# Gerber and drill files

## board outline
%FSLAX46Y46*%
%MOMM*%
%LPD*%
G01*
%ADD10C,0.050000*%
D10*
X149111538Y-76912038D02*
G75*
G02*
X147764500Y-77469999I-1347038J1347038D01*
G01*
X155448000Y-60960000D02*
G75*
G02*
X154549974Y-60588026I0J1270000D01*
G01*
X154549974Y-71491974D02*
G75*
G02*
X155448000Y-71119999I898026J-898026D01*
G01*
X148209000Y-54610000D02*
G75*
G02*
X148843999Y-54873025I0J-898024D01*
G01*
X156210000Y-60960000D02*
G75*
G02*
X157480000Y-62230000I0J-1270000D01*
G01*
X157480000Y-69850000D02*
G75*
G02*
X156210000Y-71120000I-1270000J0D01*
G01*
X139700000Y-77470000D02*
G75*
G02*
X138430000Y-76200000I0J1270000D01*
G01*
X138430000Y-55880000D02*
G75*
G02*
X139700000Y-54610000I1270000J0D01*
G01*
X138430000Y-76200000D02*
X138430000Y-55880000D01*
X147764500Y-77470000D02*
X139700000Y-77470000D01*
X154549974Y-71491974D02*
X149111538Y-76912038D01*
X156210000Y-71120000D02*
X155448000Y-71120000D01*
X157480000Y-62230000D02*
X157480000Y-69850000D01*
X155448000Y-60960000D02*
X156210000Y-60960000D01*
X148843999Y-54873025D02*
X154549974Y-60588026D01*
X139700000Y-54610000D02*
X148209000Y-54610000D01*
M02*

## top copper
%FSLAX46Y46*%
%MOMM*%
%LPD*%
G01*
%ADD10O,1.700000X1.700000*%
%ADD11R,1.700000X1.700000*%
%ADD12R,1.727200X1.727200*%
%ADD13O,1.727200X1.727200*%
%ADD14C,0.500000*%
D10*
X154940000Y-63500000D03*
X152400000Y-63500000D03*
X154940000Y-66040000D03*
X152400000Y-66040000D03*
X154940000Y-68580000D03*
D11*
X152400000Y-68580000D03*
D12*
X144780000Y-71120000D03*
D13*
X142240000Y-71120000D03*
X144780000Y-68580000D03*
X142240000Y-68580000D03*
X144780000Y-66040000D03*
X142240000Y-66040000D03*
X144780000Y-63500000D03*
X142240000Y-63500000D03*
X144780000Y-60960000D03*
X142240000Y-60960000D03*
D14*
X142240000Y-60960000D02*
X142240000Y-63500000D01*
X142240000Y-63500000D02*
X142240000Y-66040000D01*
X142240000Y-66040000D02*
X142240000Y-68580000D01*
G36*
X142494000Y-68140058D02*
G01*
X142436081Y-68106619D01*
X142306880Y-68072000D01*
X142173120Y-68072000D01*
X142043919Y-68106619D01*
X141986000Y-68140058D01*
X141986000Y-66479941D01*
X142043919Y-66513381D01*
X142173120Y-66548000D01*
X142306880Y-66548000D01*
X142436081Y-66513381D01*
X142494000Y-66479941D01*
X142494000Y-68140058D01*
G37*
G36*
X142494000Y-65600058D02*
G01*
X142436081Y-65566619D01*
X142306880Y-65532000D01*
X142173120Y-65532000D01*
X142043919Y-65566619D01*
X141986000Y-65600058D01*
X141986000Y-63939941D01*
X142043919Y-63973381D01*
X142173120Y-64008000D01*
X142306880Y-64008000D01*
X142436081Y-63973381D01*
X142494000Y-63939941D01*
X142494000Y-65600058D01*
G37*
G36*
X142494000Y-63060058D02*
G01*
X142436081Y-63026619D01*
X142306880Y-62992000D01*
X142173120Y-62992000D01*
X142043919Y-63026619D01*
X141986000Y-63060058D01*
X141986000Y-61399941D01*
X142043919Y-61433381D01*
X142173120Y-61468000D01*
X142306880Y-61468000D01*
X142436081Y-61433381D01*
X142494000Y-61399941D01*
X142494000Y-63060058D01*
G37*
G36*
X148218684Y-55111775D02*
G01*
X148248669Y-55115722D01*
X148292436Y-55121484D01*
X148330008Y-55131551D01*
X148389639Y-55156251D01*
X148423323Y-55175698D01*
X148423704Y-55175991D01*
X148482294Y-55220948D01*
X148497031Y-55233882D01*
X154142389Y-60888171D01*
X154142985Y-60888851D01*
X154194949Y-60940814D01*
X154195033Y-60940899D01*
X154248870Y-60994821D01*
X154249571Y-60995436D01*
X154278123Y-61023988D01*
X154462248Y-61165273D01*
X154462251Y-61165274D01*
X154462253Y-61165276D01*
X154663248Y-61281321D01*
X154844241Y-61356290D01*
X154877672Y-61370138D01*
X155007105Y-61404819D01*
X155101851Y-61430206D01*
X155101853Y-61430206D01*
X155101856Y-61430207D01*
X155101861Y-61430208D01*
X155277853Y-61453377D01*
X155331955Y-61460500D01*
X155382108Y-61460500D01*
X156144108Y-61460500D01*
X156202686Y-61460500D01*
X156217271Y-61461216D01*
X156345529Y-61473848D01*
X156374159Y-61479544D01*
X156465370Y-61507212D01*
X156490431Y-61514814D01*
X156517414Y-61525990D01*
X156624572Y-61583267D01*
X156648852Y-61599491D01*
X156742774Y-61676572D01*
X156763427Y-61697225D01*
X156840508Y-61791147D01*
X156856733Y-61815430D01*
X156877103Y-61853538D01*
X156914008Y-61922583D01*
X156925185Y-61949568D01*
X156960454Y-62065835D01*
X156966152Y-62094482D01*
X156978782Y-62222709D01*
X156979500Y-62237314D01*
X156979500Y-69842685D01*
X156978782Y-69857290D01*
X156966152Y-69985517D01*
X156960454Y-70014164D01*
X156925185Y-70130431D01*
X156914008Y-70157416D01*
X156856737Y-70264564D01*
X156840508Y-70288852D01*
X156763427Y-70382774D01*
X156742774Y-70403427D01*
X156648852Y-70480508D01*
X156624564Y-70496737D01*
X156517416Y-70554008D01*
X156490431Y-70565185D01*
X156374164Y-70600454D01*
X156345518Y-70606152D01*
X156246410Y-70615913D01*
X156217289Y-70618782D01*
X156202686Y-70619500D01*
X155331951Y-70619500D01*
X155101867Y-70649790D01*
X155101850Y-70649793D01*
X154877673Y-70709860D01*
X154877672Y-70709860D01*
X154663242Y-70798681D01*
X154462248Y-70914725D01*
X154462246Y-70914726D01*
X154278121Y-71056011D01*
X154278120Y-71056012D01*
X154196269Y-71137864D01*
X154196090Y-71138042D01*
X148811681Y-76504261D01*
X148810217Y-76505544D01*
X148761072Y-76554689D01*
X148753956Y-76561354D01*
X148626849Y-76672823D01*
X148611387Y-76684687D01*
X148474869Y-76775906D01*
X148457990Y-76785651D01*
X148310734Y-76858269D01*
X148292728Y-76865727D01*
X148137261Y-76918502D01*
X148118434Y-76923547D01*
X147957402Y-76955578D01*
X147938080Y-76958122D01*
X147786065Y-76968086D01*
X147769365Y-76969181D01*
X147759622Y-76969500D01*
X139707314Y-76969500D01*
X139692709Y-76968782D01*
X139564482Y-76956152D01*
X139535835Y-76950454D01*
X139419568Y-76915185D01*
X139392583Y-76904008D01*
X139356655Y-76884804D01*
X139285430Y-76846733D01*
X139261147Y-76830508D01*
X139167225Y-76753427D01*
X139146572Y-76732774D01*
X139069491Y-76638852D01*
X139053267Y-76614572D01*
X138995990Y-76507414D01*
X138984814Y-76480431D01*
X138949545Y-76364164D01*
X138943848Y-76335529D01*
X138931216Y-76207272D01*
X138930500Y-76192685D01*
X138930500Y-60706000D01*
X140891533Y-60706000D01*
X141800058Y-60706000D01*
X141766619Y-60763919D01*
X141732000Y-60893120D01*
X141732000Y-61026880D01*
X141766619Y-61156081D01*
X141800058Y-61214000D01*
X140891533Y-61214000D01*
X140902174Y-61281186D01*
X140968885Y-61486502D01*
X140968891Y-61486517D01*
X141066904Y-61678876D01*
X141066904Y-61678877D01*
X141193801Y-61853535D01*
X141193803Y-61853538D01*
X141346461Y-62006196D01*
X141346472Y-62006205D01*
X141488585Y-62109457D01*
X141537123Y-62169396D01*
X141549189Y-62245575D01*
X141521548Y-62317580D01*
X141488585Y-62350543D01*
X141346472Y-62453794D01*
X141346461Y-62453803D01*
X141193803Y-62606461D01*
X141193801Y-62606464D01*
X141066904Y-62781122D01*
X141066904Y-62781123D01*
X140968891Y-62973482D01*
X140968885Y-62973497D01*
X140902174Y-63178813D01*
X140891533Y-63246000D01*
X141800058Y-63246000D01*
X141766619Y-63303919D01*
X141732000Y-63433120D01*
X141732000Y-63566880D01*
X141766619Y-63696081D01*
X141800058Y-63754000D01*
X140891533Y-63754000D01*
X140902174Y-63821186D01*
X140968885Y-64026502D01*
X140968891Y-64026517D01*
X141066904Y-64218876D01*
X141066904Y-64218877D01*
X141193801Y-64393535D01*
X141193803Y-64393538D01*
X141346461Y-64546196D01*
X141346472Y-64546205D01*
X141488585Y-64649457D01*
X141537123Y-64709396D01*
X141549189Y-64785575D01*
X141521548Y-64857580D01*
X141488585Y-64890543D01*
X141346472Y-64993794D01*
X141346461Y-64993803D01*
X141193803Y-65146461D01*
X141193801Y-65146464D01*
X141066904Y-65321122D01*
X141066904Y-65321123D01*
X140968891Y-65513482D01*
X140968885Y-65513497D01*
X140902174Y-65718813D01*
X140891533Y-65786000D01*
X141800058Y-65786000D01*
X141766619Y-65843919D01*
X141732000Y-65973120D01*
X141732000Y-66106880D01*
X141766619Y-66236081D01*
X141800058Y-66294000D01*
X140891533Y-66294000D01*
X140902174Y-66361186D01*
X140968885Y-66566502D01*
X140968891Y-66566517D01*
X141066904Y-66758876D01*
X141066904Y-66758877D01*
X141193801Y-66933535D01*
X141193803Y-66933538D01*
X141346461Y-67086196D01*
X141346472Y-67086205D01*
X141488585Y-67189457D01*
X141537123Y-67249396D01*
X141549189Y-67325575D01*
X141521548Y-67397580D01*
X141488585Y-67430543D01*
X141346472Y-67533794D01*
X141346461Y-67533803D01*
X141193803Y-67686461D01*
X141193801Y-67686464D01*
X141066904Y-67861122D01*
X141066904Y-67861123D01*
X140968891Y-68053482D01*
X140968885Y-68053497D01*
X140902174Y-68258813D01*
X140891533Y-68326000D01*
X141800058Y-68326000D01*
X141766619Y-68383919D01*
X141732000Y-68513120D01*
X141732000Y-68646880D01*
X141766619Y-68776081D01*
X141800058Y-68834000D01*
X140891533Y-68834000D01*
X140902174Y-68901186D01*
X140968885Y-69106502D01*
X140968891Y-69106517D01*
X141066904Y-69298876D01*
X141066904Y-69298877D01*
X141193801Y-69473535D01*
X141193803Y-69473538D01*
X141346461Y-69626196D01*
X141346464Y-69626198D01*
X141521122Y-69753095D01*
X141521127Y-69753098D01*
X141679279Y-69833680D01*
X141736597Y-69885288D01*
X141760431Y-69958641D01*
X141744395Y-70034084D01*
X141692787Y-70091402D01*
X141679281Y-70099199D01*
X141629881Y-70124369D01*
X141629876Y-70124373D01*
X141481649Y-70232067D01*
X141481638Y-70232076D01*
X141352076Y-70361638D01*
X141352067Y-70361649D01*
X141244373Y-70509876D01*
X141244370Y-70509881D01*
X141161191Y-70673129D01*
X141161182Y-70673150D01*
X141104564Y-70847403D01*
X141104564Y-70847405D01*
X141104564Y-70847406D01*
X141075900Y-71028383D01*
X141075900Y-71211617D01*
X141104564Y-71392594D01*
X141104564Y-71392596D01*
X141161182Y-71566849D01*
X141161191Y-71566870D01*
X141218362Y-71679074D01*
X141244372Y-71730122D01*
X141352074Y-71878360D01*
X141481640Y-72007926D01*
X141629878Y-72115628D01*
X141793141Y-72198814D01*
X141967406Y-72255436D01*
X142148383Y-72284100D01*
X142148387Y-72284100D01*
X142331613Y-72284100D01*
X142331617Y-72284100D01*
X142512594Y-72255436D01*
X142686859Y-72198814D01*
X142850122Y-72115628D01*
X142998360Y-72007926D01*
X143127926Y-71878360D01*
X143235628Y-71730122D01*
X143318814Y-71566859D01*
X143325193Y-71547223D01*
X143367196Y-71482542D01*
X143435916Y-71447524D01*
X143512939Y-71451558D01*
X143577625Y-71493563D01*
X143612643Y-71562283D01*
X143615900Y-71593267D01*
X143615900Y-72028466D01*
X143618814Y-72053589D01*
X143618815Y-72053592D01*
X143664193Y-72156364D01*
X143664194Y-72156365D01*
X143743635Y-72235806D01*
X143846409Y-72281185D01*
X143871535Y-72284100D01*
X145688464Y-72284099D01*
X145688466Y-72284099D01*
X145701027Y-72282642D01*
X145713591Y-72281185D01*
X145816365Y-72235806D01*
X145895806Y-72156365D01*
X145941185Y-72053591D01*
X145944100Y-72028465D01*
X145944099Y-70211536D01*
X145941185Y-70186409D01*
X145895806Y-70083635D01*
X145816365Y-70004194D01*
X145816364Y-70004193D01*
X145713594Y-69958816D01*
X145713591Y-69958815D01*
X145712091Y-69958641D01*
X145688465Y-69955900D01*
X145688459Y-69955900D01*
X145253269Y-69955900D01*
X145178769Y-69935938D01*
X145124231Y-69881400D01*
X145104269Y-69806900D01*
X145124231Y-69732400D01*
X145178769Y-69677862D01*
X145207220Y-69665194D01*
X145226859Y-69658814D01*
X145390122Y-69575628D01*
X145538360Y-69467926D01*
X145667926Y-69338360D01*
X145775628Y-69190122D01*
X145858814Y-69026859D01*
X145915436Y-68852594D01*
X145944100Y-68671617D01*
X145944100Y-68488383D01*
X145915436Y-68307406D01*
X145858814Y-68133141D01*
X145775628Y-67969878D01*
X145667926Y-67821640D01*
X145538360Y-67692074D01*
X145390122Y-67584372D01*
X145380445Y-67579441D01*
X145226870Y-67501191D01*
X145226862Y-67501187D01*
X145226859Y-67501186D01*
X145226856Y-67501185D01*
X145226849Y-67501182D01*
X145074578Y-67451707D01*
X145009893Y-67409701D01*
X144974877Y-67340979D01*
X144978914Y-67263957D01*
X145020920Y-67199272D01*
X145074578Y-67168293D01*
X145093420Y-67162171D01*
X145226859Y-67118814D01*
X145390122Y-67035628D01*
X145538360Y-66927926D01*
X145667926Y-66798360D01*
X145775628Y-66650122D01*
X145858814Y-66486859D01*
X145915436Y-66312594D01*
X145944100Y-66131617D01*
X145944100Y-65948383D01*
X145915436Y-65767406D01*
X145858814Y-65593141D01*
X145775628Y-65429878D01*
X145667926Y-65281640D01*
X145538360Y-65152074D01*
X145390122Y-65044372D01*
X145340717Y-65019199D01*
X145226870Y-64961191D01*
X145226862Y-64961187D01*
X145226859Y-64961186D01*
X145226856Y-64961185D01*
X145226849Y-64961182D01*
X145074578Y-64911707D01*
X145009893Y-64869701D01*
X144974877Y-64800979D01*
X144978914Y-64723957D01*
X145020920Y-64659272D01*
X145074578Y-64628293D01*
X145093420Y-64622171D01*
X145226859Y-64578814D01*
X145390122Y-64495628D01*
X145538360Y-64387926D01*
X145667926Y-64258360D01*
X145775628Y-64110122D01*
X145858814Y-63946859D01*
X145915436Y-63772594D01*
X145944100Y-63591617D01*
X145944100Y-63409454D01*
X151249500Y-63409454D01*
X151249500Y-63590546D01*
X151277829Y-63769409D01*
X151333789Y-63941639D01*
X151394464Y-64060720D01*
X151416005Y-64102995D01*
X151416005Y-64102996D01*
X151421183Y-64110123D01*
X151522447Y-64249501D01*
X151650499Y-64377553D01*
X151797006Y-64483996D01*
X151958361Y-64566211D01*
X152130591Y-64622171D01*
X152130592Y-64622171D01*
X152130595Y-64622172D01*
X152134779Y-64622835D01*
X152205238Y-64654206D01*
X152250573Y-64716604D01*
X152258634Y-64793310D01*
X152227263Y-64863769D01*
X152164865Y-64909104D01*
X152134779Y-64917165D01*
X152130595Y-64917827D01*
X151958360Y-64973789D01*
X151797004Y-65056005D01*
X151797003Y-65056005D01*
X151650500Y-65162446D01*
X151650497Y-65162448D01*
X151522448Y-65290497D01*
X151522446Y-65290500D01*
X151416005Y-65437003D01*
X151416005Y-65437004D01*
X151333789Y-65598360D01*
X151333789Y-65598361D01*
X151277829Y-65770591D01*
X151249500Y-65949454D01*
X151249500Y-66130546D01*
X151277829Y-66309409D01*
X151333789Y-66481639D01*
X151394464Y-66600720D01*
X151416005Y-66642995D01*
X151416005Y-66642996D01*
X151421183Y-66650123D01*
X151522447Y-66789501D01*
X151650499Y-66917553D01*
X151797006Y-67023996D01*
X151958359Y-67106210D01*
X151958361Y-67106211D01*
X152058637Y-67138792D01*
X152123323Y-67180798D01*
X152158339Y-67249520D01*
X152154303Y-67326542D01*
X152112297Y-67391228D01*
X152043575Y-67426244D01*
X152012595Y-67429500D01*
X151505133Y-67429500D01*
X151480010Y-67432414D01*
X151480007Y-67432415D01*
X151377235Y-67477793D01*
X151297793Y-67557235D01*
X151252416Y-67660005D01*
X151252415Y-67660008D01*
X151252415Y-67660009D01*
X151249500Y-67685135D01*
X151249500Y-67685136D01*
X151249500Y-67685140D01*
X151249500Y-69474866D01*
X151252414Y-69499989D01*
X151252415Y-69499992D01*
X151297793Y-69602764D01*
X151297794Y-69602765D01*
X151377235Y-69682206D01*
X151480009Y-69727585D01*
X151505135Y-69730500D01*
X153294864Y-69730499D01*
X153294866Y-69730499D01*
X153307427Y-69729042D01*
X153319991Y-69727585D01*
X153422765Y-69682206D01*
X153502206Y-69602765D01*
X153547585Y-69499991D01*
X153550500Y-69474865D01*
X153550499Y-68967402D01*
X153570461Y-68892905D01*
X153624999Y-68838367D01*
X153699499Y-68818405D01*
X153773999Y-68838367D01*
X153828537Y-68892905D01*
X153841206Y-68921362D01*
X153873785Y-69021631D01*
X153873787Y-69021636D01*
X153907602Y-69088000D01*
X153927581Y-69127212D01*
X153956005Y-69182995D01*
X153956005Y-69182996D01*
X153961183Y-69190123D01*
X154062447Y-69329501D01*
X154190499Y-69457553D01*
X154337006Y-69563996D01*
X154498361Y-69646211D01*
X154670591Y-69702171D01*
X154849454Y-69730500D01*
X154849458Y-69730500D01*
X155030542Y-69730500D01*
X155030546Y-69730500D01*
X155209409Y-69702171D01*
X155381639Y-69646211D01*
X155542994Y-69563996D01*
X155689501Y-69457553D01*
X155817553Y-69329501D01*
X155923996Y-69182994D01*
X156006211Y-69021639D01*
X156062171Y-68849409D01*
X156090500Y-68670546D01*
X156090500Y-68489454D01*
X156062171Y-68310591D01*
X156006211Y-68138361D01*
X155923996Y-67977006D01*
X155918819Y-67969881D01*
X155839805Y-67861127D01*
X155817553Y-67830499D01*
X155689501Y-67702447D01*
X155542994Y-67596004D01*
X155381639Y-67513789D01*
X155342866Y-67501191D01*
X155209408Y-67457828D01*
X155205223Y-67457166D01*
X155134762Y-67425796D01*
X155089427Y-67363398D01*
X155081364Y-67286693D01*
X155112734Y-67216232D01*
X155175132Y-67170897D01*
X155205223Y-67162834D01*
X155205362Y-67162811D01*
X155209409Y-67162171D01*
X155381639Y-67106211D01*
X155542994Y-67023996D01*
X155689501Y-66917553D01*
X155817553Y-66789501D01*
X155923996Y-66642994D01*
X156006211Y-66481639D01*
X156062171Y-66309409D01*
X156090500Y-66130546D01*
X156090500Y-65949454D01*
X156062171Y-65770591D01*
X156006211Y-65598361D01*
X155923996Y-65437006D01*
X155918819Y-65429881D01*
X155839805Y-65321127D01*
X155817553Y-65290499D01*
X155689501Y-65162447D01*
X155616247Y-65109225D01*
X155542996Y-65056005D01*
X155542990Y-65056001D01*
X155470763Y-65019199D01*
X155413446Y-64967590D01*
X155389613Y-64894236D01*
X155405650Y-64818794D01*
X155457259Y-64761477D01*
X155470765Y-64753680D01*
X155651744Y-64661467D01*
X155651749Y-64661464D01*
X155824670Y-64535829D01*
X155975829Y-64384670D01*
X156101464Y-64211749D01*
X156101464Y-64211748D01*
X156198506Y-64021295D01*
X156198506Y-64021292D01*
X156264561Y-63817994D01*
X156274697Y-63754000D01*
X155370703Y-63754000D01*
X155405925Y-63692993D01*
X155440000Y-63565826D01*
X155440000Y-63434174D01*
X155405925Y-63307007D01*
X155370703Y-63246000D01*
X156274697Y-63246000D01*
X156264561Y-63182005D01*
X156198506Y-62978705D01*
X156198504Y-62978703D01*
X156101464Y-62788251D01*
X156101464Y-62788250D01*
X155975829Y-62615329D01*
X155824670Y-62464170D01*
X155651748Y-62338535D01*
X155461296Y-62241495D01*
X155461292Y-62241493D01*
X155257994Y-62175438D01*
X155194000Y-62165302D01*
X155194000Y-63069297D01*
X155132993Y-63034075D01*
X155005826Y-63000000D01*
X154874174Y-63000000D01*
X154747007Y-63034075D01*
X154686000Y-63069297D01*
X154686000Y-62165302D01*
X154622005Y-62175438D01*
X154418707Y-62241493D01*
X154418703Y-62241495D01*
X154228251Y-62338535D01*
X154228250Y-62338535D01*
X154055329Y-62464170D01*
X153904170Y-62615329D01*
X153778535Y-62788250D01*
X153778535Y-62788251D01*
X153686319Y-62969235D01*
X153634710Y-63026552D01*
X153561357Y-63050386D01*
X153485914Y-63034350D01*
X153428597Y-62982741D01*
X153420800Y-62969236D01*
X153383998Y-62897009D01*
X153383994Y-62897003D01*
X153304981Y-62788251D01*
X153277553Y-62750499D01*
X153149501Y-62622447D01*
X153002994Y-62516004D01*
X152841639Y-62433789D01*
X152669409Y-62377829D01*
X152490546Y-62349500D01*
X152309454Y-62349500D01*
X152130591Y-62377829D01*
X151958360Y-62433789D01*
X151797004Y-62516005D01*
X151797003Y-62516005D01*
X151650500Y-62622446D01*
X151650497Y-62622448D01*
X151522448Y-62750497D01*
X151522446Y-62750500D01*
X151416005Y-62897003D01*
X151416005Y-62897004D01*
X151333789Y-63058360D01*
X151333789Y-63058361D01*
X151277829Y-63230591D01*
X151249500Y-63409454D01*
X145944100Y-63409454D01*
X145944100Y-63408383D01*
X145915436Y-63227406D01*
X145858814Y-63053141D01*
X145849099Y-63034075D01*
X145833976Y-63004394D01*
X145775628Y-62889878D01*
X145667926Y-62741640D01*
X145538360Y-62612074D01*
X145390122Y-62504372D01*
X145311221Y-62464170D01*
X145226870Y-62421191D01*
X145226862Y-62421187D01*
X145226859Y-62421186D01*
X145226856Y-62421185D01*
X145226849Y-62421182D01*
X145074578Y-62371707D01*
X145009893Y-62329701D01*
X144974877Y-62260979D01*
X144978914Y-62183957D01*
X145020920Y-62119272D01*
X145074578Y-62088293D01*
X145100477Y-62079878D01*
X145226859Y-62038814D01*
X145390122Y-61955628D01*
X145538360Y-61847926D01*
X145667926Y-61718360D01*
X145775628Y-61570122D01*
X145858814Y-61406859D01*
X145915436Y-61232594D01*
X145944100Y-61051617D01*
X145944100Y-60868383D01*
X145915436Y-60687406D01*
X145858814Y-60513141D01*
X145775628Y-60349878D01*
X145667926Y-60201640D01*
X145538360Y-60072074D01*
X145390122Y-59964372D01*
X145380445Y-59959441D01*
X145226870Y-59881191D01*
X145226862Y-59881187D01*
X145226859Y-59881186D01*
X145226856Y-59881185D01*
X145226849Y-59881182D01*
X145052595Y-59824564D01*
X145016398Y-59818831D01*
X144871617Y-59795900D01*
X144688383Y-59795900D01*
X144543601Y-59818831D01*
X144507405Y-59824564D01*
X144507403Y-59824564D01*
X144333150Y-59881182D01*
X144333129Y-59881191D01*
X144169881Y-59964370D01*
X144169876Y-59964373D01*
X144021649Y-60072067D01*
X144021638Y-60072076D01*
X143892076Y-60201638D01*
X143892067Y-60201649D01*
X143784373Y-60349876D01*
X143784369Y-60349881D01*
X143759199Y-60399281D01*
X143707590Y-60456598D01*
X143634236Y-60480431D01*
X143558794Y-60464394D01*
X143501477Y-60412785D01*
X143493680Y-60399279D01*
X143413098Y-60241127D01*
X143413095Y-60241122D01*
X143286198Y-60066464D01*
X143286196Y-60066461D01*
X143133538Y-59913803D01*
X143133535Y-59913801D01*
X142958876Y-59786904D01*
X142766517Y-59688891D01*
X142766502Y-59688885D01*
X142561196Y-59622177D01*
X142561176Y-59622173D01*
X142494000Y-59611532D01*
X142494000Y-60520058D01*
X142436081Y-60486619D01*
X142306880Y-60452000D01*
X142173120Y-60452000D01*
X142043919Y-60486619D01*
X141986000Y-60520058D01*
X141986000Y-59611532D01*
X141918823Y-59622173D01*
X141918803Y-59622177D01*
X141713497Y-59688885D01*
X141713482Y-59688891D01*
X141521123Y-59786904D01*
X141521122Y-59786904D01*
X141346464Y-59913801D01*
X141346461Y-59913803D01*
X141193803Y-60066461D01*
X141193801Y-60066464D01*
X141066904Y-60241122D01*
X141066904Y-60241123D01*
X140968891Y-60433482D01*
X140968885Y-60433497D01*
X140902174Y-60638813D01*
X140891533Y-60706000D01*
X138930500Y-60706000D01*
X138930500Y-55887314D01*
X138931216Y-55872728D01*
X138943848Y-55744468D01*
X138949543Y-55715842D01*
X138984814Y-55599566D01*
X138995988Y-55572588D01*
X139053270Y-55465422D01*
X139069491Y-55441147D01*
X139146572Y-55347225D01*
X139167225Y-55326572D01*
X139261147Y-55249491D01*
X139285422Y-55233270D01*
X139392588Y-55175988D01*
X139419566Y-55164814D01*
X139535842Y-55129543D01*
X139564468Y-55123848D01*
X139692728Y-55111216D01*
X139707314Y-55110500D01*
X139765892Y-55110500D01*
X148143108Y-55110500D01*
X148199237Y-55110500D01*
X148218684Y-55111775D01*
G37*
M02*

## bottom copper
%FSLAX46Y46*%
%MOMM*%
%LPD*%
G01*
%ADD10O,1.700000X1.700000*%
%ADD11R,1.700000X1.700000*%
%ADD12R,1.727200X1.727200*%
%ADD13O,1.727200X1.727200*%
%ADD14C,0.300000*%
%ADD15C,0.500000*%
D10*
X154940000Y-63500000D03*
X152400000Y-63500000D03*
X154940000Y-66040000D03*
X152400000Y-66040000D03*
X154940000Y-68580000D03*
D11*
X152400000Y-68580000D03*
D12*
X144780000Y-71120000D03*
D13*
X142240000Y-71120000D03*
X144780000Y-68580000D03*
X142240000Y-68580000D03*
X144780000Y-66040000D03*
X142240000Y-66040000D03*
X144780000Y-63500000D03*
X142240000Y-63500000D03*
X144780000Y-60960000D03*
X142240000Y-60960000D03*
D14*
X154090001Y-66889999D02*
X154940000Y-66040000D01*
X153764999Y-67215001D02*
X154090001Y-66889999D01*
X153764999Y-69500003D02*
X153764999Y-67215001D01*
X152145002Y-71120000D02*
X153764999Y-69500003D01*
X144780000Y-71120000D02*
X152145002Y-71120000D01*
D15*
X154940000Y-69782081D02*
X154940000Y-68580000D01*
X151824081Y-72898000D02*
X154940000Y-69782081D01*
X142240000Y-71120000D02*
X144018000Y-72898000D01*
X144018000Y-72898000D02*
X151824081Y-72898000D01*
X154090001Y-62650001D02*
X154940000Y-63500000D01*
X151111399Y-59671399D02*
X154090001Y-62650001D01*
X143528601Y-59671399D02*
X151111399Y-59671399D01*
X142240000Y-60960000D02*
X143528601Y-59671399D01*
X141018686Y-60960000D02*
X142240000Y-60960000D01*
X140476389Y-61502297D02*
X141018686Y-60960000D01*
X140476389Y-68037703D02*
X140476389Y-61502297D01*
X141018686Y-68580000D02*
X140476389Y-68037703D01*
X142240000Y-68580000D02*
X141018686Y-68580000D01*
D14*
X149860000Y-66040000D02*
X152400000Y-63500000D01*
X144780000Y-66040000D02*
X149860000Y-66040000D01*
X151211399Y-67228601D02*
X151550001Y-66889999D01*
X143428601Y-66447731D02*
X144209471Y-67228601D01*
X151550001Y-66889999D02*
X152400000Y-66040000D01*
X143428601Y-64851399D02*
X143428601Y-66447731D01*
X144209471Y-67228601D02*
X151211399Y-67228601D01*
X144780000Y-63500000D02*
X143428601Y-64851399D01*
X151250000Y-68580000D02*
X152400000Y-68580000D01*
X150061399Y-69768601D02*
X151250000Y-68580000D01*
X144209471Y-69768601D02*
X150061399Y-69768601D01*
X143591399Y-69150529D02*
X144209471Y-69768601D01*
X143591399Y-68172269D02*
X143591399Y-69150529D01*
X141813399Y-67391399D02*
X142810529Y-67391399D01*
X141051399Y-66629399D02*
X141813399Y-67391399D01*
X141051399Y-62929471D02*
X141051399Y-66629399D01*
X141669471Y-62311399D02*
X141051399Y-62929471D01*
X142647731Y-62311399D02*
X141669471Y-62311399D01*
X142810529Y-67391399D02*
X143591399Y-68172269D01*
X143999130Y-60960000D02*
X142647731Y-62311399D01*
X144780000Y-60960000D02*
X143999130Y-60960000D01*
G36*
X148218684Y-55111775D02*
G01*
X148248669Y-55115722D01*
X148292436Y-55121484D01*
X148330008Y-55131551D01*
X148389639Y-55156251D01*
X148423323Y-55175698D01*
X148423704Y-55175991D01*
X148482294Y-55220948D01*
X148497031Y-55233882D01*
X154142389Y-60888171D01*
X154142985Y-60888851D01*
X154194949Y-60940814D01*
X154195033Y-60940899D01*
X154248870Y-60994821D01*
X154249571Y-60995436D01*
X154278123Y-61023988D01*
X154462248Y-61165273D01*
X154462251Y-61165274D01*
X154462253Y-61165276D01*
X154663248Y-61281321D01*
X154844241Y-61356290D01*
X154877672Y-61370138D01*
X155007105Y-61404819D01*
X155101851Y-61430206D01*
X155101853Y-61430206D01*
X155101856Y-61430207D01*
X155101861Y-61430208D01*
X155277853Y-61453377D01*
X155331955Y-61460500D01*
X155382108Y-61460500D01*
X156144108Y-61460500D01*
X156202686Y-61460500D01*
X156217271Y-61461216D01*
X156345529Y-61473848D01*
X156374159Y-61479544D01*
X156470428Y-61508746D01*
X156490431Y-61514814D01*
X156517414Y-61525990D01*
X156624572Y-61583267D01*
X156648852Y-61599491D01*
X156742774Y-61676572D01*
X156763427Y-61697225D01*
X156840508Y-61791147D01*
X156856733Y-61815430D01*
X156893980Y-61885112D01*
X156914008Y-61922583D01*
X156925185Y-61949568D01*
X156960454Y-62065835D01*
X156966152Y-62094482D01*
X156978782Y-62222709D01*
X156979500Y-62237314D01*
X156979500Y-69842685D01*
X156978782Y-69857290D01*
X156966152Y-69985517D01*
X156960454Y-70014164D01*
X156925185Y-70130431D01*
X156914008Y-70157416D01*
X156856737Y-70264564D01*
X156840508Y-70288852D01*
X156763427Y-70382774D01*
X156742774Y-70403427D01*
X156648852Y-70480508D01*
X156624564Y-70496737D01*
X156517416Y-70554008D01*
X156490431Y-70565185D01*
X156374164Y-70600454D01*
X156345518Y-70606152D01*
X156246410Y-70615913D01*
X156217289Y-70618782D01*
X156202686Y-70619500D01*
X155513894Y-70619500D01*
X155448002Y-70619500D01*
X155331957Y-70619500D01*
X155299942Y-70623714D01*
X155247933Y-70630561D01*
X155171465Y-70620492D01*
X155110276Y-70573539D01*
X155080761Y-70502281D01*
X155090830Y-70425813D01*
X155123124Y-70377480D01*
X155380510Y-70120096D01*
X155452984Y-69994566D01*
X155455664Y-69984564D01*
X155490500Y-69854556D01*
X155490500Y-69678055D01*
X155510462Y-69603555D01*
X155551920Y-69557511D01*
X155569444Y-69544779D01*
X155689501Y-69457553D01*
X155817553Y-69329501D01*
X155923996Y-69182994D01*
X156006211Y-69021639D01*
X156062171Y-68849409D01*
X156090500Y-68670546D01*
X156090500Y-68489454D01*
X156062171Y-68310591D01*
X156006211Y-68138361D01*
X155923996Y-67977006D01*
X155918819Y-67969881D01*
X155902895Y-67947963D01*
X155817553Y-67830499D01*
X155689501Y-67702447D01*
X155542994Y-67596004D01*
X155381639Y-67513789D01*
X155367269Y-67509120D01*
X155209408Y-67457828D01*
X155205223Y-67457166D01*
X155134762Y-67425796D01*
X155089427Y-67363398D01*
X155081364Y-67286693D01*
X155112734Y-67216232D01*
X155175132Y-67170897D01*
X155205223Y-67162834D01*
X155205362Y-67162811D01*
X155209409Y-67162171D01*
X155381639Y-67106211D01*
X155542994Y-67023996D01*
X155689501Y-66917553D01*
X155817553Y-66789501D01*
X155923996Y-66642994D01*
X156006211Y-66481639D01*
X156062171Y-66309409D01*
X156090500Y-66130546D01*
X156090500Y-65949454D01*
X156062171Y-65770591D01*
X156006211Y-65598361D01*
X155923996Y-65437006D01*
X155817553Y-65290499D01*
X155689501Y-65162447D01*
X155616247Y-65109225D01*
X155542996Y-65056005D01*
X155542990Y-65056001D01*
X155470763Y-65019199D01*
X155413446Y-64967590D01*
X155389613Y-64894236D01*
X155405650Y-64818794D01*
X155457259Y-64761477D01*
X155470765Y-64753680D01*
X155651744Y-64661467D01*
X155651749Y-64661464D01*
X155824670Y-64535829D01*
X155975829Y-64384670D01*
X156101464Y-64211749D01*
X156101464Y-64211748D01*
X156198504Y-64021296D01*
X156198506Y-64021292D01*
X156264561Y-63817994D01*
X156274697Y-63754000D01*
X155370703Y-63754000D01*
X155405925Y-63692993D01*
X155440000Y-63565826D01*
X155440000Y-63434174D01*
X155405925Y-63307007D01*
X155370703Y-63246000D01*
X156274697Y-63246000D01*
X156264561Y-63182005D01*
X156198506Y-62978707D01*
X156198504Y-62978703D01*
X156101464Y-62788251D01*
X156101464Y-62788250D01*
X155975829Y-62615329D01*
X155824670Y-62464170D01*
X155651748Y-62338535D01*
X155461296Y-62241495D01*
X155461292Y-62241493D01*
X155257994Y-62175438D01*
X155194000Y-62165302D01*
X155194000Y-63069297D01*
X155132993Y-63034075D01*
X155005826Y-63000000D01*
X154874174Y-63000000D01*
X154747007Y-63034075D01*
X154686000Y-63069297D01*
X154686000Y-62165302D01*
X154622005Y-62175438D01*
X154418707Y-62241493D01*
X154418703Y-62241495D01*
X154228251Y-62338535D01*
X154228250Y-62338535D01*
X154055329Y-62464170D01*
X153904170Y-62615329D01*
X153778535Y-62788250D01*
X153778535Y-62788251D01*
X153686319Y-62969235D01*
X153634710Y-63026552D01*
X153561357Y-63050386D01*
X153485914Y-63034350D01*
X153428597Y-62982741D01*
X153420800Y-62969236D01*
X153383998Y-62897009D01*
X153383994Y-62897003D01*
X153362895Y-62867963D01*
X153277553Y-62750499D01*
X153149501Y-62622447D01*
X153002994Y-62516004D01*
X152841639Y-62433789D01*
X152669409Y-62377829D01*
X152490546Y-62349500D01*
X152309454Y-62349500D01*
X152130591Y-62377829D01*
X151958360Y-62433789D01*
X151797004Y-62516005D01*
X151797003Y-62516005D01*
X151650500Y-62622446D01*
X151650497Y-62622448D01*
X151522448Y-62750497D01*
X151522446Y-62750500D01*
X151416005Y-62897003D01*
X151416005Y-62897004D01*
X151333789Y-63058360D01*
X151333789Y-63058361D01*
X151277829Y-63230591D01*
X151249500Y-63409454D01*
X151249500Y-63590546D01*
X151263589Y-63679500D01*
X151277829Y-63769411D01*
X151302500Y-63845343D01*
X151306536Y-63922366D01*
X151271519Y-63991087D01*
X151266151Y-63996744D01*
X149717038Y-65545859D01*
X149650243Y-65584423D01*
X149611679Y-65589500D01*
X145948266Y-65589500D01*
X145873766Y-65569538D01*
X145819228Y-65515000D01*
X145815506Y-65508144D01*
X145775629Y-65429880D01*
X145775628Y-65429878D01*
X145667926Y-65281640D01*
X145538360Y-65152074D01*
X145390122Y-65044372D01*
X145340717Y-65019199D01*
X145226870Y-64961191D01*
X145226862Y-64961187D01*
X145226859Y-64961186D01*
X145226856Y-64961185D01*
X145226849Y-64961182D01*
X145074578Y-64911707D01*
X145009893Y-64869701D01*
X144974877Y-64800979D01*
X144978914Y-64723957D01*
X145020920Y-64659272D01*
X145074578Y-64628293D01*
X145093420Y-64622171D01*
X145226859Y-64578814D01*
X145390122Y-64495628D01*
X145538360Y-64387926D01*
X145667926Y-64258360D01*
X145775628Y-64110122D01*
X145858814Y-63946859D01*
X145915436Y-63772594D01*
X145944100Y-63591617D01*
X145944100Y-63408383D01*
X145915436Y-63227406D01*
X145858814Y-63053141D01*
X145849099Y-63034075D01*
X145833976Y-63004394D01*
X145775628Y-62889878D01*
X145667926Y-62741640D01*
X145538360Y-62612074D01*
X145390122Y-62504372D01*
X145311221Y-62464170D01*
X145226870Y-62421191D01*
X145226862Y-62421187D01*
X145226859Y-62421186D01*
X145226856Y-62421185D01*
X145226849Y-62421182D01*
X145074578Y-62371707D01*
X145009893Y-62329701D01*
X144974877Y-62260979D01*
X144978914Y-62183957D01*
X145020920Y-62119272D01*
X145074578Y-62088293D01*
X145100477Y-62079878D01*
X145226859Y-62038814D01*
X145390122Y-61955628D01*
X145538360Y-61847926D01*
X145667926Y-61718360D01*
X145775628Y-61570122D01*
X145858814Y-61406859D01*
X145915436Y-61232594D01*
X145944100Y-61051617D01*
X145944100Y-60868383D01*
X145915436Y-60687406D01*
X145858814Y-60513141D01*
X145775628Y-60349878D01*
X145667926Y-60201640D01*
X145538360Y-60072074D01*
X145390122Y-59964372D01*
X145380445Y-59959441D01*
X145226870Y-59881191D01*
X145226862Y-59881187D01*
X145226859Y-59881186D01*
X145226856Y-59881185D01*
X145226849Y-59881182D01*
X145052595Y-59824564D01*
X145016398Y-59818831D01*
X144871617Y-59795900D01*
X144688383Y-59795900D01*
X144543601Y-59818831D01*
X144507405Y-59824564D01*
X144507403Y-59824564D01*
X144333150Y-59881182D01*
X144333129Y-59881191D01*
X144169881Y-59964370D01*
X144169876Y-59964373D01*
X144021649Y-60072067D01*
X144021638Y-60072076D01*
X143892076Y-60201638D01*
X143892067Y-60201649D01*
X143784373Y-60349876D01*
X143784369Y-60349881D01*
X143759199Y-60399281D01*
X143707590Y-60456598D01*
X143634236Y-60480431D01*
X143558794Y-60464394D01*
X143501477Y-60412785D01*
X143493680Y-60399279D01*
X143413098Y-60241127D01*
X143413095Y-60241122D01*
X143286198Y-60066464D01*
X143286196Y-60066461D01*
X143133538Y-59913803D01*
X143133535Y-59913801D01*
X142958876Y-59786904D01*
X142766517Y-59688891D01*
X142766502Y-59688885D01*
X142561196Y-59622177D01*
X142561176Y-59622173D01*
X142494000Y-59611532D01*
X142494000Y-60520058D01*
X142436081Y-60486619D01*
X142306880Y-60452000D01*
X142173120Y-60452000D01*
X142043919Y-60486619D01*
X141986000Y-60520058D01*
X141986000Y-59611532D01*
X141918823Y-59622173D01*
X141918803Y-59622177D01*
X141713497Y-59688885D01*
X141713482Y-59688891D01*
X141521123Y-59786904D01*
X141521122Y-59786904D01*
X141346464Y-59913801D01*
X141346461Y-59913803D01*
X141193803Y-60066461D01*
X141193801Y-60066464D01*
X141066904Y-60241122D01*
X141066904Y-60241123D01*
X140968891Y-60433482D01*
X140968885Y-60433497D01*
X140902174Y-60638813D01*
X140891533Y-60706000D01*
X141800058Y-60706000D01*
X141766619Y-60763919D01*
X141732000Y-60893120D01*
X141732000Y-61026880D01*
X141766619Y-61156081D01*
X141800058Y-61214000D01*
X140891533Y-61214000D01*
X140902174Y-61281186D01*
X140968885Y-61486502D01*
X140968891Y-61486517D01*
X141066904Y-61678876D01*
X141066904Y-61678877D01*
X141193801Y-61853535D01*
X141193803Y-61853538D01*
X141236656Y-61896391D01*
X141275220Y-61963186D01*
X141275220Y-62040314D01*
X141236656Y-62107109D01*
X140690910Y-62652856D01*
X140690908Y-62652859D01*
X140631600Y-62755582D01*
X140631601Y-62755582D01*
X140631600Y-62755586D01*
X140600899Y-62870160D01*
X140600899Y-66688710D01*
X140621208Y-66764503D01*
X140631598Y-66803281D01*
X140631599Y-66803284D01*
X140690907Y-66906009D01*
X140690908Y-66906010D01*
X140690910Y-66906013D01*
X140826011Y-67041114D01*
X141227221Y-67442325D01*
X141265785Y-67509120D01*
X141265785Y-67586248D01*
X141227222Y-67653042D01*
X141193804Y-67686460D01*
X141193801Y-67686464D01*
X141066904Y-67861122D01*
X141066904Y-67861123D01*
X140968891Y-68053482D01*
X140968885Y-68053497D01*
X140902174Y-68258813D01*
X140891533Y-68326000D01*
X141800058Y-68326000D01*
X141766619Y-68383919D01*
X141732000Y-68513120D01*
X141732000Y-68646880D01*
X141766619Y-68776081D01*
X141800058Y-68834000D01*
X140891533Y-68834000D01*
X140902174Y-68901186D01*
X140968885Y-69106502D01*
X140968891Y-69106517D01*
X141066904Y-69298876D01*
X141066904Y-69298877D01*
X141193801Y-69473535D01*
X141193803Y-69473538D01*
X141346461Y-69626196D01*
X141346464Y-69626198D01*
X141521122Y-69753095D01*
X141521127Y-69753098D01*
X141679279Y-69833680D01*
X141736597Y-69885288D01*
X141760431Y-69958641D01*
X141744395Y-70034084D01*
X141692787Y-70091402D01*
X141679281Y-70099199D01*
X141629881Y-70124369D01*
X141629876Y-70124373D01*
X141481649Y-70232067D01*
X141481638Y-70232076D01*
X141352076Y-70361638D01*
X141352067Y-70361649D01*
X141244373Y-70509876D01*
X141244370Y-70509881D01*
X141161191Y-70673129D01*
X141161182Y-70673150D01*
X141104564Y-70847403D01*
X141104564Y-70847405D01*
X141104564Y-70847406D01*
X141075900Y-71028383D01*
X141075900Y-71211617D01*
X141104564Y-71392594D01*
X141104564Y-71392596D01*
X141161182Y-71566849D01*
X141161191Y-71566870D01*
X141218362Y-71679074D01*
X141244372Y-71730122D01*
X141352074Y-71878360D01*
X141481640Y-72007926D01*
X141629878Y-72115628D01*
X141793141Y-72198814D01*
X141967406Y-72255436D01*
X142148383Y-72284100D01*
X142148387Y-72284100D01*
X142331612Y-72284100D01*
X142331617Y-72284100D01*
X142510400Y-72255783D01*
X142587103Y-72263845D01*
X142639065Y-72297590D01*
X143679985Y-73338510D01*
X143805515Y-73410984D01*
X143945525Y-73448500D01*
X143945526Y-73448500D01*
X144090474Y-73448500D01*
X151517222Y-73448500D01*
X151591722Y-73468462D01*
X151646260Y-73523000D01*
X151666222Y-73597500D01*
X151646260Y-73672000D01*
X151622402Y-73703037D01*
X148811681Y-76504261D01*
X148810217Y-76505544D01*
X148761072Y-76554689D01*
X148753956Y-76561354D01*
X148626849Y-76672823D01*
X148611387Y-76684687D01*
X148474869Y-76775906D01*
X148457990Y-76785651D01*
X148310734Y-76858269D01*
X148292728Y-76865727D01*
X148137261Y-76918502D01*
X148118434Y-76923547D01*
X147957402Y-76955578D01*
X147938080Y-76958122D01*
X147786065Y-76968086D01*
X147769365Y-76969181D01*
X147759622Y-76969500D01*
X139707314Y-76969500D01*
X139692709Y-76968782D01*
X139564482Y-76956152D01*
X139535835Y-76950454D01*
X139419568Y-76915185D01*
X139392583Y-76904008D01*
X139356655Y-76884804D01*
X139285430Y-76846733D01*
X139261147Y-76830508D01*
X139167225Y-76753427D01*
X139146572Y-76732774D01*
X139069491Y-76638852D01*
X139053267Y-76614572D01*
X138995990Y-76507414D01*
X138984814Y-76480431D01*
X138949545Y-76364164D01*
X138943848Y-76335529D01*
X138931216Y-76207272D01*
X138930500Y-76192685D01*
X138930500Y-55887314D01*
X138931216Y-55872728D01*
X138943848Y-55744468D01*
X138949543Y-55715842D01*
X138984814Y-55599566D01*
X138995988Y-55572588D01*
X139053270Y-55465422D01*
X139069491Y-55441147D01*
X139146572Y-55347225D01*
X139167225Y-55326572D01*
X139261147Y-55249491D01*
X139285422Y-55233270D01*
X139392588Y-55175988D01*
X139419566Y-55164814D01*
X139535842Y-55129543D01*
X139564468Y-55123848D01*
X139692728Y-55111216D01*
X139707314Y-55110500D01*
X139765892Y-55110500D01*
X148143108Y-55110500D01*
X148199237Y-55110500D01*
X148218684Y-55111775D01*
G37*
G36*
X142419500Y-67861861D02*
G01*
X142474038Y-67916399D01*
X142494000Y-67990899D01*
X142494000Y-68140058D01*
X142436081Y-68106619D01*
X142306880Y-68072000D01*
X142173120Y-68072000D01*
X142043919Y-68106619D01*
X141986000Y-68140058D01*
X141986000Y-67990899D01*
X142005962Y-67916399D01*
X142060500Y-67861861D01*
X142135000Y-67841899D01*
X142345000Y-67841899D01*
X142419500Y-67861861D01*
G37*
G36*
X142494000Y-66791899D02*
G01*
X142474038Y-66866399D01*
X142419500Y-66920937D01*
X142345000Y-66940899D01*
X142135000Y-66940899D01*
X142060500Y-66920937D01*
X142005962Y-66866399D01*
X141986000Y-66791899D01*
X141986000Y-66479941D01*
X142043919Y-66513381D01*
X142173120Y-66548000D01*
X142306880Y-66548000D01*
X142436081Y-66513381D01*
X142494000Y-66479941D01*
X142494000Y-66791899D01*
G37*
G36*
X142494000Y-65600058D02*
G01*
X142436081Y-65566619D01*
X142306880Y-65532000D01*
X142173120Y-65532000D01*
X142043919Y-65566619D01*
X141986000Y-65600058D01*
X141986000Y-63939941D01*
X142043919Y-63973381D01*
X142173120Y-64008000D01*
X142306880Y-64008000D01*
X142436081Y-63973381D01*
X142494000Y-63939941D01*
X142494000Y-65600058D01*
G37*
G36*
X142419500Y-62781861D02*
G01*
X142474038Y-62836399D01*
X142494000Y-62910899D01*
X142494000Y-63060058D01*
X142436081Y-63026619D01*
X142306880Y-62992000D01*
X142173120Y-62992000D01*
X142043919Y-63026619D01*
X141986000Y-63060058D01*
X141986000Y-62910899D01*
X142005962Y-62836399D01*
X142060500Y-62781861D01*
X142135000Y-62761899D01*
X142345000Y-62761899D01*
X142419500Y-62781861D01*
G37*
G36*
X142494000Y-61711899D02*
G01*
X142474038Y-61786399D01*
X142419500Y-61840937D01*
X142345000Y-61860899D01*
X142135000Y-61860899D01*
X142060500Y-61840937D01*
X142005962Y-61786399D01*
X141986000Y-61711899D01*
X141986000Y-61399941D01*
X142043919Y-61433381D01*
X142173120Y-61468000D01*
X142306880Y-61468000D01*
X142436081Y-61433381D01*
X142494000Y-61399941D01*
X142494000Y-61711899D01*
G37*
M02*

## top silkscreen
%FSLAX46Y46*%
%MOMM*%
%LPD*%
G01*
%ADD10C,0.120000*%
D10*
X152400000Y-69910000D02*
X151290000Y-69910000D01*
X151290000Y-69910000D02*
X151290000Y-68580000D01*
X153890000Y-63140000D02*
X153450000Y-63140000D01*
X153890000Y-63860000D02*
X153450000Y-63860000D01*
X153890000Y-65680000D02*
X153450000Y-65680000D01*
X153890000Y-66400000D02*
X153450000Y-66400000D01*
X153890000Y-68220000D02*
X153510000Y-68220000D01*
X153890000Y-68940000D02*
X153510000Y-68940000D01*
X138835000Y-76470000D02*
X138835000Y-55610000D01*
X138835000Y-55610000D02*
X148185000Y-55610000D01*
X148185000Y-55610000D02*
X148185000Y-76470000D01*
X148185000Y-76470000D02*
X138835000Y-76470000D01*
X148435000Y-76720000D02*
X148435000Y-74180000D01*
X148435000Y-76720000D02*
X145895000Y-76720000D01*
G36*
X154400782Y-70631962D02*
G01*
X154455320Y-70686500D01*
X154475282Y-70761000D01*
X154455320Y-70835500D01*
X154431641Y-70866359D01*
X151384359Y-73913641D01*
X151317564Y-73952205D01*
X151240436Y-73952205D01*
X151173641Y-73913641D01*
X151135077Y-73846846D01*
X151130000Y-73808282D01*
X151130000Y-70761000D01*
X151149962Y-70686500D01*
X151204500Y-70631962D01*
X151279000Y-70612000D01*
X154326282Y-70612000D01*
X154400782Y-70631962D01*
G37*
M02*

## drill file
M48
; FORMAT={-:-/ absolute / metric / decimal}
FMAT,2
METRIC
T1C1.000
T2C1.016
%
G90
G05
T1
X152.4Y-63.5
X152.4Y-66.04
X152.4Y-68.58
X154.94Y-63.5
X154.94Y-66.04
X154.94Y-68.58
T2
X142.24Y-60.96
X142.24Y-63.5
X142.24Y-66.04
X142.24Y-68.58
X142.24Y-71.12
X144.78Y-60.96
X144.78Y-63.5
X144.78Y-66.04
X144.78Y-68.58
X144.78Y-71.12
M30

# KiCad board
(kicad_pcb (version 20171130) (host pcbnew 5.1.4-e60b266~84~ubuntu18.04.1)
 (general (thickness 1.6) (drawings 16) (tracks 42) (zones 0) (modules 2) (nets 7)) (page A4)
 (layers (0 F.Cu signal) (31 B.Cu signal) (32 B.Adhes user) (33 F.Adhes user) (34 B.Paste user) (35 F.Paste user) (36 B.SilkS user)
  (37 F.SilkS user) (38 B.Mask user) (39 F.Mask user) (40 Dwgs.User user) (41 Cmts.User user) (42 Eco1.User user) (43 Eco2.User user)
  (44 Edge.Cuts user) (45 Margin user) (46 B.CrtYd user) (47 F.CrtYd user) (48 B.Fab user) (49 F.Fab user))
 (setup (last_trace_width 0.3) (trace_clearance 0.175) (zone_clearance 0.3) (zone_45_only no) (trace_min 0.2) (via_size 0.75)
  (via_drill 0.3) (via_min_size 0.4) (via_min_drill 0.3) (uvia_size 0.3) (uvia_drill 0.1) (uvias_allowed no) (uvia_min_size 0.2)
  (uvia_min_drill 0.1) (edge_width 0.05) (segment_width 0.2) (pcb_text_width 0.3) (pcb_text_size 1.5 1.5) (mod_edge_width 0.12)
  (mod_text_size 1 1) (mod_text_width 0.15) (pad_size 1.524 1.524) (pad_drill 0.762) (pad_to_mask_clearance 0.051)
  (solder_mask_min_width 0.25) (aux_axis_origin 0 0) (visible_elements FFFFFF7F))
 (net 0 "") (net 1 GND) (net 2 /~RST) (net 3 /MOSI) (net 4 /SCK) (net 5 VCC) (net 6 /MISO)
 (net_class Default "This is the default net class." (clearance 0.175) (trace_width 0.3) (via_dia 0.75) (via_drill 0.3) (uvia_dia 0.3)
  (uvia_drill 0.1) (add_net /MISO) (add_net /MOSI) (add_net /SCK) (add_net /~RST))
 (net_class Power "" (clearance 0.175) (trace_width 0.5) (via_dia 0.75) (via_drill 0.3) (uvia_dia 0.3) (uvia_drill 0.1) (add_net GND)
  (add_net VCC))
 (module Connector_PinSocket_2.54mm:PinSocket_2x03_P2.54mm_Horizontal (layer F.Cu) (at 152.4 68.58 180)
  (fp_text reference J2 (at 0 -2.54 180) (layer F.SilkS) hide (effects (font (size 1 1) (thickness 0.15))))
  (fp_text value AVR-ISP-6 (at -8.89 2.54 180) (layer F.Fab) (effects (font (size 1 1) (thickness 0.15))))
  (fp_line (start 0 -1.33) (end 1.11 -1.33) (layer F.SilkS) (width 0.12))
  (fp_line (start 1.11 -1.33) (end 1.11 0) (layer F.SilkS) (width 0.12))
  (fp_line (start -1.49 5.44) (end -1.05 5.44) (layer F.SilkS) (width 0.12))
  (fp_line (start -1.49 4.72) (end -1.05 4.72) (layer F.SilkS) (width 0.12))
  (fp_line (start -1.49 2.9) (end -1.05 2.9) (layer F.SilkS) (width 0.12))
  (fp_line (start -1.49 2.18) (end -1.05 2.18) (layer F.SilkS) (width 0.12))
  (fp_line (start -1.49 0.36) (end -1.11 0.36) (layer F.SilkS) (width 0.12))
  (fp_line (start -1.49 -0.36) (end -1.11 -0.36) (layer F.SilkS) (width 0.12))
  (pad 6 thru_hole oval (at -2.54 5.08 180) (size 1.7 1.7) (drill 1) (layers *.Cu *.Mask) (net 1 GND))
  (pad 5 thru_hole oval (at 0 5.08 180) (size 1.7 1.7) (drill 1) (layers *.Cu *.Mask) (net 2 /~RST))
  (pad 4 thru_hole oval (at -2.54 2.54 180) (size 1.7 1.7) (drill 1) (layers *.Cu *.Mask) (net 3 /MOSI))
  (pad 3 thru_hole oval (at 0 2.54 180) (size 1.7 1.7) (drill 1) (layers *.Cu *.Mask) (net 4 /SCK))
  (pad 2 thru_hole oval (at -2.54 0 180) (size 1.7 1.7) (drill 1) (layers *.Cu *.Mask) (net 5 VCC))
  (pad 1 thru_hole rect (at 0 0 180) (size 1.7 1.7) (drill 1) (layers *.Cu *.Mask) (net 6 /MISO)))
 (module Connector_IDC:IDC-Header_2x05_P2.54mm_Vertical (layer F.Cu) (at 144.78 71.12 180)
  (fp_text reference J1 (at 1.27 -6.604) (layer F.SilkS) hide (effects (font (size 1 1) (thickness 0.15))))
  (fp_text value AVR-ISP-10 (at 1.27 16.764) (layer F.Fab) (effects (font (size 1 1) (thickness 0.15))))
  (fp_line (start 5.945 -5.35) (end 5.945 15.51) (layer F.SilkS) (width 0.12))
  (fp_line (start 5.945 15.51) (end -3.405 15.51) (layer F.SilkS) (width 0.12))
  (fp_line (start -3.405 15.51) (end -3.405 -5.35) (layer F.SilkS) (width 0.12))
  (fp_line (start -3.405 -5.35) (end 5.945 -5.35) (layer F.SilkS) (width 0.12))
  (fp_line (start -3.655 -5.6) (end -3.655 -3.06) (layer F.SilkS) (width 0.12))
  (fp_line (start -3.655 -5.6) (end -1.115 -5.6) (layer F.SilkS) (width 0.12))
  (pad 1 thru_hole rect (at 0 0 180) (size 1.7272 1.7272) (drill 1.016) (layers *.Cu *.Mask) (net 3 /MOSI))
  (pad 2 thru_hole oval (at 2.54 0 180) (size 1.7272 1.7272) (drill 1.016) (layers *.Cu *.Mask) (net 5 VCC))
  (pad 3 thru_hole oval (at 0 2.54 180) (size 1.7272 1.7272) (drill 1.016) (layers *.Cu *.Mask))
  (pad 4 thru_hole oval (at 2.54 2.54 180) (size 1.7272 1.7272) (drill 1.016) (layers *.Cu *.Mask) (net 1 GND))
  (pad 5 thru_hole oval (at 0 5.08 180) (size 1.7272 1.7272) (drill 1.016) (layers *.Cu *.Mask) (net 2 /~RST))
  (pad 6 thru_hole oval (at 2.54 5.08 180) (size 1.7272 1.7272) (drill 1.016) (layers *.Cu *.Mask) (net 1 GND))
  (pad 7 thru_hole oval (at 0 7.62 180) (size 1.7272 1.7272) (drill 1.016) (layers *.Cu *.Mask) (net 4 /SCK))
  (pad 8 thru_hole oval (at 2.54 7.62 180) (size 1.7272 1.7272) (drill 1.016) (layers *.Cu *.Mask) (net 1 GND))
  (pad 9 thru_hole oval (at 0 10.16 180) (size 1.7272 1.7272) (drill 1.016) (layers *.Cu *.Mask) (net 6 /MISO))
  (pad 10 thru_hole oval (at 2.54 10.16 180) (size 1.7272 1.7272) (drill 1.016) (layers *.Cu *.Mask) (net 1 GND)))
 (gr_arc (start 147.7645 75.565) (end 147.7645 77.47) (angle -45) (layer Edge.Cuts) (width 0.05))
 (gr_arc (start 155.448 59.69) (end 155.448 60.96) (angle 45) (layer Edge.Cuts) (width 0.05))
 (gr_arc (start 155.448 72.39) (end 155.448 71.12) (angle -45) (layer Edge.Cuts) (width 0.05))
 (gr_arc (start 148.209 55.508024) (end 148.843999 54.873025) (angle -45) (layer Edge.Cuts) (width 0.05))
 (gr_arc (start 156.21 62.23) (end 157.48 62.23) (angle -90) (layer Edge.Cuts) (width 0.05))
 (gr_arc (start 156.21 69.85) (end 156.21 71.12) (angle -90) (layer Edge.Cuts) (width 0.05))
 (gr_arc (start 139.7 76.2) (end 138.43 76.2) (angle -90) (layer Edge.Cuts) (width 0.05))
 (gr_arc (start 139.7 55.88) (end 139.7 54.61) (angle -90) (layer Edge.Cuts) (width 0.05))
 (gr_line (start 138.43 76.2) (end 138.43 55.88) (layer Edge.Cuts) (width 0.05))
 (gr_line (start 147.7645 77.47) (end 139.7 77.47) (layer Edge.Cuts) (width 0.05))
 (gr_line (start 154.549974 71.491974) (end 149.111538 76.912038) (layer Edge.Cuts) (width 0.05))
 (gr_line (start 156.21 71.12) (end 155.448 71.12) (layer Edge.Cuts) (width 0.05))
 (gr_line (start 157.48 62.23) (end 157.48 69.85) (layer Edge.Cuts) (width 0.05))
 (gr_line (start 155.448 60.96) (end 156.21 60.96) (layer Edge.Cuts) (width 0.05))
 (gr_line (start 148.843999 54.873025) (end 154.549974 60.588026) (layer Edge.Cuts) (width 0.05))
 (gr_line (start 139.7 54.61) (end 148.209 54.61) (layer Edge.Cuts) (width 0.05))
 (segment (start 154.090001 66.889999) (end 154.94 66.04) (width 0.3) (layer B.Cu) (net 3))
 (segment (start 153.764999 67.215001) (end 154.090001 66.889999) (width 0.3) (layer B.Cu) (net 3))
 (segment (start 153.764999 69.500003) (end 153.764999 67.215001) (width 0.3) (layer B.Cu) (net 3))
 (segment (start 152.145002 71.12) (end 153.764999 69.500003) (width 0.3) (layer B.Cu) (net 3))
 (segment (start 144.78 71.12) (end 152.145002 71.12) (width 0.3) (layer B.Cu) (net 3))
 (segment (start 154.94 69.782081) (end 154.94 68.58) (width 0.5) (layer B.Cu) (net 5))
 (segment (start 151.824081 72.898) (end 154.94 69.782081) (width 0.5) (layer B.Cu) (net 5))
 (segment (start 142.24 71.12) (end 144.018 72.898) (width 0.5) (layer B.Cu) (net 5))
 (segment (start 144.018 72.898) (end 151.824081 72.898) (width 0.5) (layer B.Cu) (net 5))
 (segment (start 154.090001 62.650001) (end 154.94 63.5) (width 0.5) (layer B.Cu) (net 1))
 (segment (start 151.111399 59.671399) (end 154.090001 62.650001) (width 0.5) (layer B.Cu) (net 1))
 (segment (start 143.528601 59.671399) (end 151.111399 59.671399) (width 0.5) (layer B.Cu) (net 1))
 (segment (start 142.24 60.96) (end 143.528601 59.671399) (width 0.5) (layer B.Cu) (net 1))
 (segment (start 141.018686 60.96) (end 142.24 60.96) (width 0.5) (layer B.Cu) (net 1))
 (segment (start 140.476389 61.502297) (end 141.018686 60.96) (width 0.5) (layer B.Cu) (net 1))
 (segment (start 140.476389 68.037703) (end 140.476389 61.502297) (width 0.5) (layer B.Cu) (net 1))
 (segment (start 141.018686 68.58) (end 140.476389 68.037703) (width 0.5) (layer B.Cu) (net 1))
 (segment (start 142.24 68.58) (end 141.018686 68.58) (width 0.5) (layer B.Cu) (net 1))
 (segment (start 142.24 60.96) (end 142.24 63.5) (width 0.5) (layer F.Cu) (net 1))
 (segment (start 142.24 63.5) (end 142.24 66.04) (width 0.5) (layer F.Cu) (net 1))
 (segment (start 142.24 66.04) (end 142.24 68.58) (width 0.5) (layer F.Cu) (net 1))
 (segment (start 149.86 66.04) (end 152.4 63.5) (width 0.3) (layer B.Cu) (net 2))
 (segment (start 144.78 66.04) (end 149.86 66.04) (width 0.3) (layer B.Cu) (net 2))
 (segment (start 151.211399 67.228601) (end 151.550001 66.889999) (width 0.3) (layer B.Cu) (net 4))
 (segment (start 143.428601 66.447731) (end 144.209471 67.228601) (width 0.3) (layer B.Cu) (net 4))
 (segment (start 151.550001 66.889999) (end 152.4 66.04) (width 0.3) (layer B.Cu) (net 4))
 (segment (start 143.428601 64.851399) (end 143.428601 66.447731) (width 0.3) (layer B.Cu) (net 4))
 (segment (start 144.209471 67.228601) (end 151.211399 67.228601) (width 0.3) (layer B.Cu) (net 4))
 (segment (start 144.78 63.5) (end 143.428601 64.851399) (width 0.3) (layer B.Cu) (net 4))
 (segment (start 151.25 68.58) (end 152.4 68.58) (width 0.3) (layer B.Cu) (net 6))
 (segment (start 150.061399 69.768601) (end 151.25 68.58) (width 0.3) (layer B.Cu) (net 6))
 (segment (start 144.209471 69.768601) (end 150.061399 69.768601) (width 0.3) (layer B.Cu) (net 6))
 (segment (start 143.591399 69.150529) (end 144.209471 69.768601) (width 0.3) (layer B.Cu) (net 6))
 (segment (start 143.591399 68.172269) (end 143.591399 69.150529) (width 0.3) (layer B.Cu) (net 6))
 (segment (start 141.813399 67.391399) (end 142.810529 67.391399) (width 0.3) (layer B.Cu) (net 6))
 (segment (start 141.051399 66.629399) (end 141.813399 67.391399) (width 0.3) (layer B.Cu) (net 6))
 (segment (start 141.051399 62.929471) (end 141.051399 66.629399) (width 0.3) (layer B.Cu) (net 6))
 (segment (start 141.669471 62.311399) (end 141.051399 62.929471) (width 0.3) (layer B.Cu) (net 6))
 (segment (start 142.647731 62.311399) (end 141.669471 62.311399) (width 0.3) (layer B.Cu) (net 6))
 (segment (start 142.810529 67.391399) (end 143.591399 68.172269) (width 0.3) (layer B.Cu) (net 6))
 (segment (start 143.99913 60.96) (end 142.647731 62.311399) (width 0.3) (layer B.Cu) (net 6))
 (segment (start 144.78 60.96) (end 143.99913 60.96) (width 0.3) (layer B.Cu) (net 6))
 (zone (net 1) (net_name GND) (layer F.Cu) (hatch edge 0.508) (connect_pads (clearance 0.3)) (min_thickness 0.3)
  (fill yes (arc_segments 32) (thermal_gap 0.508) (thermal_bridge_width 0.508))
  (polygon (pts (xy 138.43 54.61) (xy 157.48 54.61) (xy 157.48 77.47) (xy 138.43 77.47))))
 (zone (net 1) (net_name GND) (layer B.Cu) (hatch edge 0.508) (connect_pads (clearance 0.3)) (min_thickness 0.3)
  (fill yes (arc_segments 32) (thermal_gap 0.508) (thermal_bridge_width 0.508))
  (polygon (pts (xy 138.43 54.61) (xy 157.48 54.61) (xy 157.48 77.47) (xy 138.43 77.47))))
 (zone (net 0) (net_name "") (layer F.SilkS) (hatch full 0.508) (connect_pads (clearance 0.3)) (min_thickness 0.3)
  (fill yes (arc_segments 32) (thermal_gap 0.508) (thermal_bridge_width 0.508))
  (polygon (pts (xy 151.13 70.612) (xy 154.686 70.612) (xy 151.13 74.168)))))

